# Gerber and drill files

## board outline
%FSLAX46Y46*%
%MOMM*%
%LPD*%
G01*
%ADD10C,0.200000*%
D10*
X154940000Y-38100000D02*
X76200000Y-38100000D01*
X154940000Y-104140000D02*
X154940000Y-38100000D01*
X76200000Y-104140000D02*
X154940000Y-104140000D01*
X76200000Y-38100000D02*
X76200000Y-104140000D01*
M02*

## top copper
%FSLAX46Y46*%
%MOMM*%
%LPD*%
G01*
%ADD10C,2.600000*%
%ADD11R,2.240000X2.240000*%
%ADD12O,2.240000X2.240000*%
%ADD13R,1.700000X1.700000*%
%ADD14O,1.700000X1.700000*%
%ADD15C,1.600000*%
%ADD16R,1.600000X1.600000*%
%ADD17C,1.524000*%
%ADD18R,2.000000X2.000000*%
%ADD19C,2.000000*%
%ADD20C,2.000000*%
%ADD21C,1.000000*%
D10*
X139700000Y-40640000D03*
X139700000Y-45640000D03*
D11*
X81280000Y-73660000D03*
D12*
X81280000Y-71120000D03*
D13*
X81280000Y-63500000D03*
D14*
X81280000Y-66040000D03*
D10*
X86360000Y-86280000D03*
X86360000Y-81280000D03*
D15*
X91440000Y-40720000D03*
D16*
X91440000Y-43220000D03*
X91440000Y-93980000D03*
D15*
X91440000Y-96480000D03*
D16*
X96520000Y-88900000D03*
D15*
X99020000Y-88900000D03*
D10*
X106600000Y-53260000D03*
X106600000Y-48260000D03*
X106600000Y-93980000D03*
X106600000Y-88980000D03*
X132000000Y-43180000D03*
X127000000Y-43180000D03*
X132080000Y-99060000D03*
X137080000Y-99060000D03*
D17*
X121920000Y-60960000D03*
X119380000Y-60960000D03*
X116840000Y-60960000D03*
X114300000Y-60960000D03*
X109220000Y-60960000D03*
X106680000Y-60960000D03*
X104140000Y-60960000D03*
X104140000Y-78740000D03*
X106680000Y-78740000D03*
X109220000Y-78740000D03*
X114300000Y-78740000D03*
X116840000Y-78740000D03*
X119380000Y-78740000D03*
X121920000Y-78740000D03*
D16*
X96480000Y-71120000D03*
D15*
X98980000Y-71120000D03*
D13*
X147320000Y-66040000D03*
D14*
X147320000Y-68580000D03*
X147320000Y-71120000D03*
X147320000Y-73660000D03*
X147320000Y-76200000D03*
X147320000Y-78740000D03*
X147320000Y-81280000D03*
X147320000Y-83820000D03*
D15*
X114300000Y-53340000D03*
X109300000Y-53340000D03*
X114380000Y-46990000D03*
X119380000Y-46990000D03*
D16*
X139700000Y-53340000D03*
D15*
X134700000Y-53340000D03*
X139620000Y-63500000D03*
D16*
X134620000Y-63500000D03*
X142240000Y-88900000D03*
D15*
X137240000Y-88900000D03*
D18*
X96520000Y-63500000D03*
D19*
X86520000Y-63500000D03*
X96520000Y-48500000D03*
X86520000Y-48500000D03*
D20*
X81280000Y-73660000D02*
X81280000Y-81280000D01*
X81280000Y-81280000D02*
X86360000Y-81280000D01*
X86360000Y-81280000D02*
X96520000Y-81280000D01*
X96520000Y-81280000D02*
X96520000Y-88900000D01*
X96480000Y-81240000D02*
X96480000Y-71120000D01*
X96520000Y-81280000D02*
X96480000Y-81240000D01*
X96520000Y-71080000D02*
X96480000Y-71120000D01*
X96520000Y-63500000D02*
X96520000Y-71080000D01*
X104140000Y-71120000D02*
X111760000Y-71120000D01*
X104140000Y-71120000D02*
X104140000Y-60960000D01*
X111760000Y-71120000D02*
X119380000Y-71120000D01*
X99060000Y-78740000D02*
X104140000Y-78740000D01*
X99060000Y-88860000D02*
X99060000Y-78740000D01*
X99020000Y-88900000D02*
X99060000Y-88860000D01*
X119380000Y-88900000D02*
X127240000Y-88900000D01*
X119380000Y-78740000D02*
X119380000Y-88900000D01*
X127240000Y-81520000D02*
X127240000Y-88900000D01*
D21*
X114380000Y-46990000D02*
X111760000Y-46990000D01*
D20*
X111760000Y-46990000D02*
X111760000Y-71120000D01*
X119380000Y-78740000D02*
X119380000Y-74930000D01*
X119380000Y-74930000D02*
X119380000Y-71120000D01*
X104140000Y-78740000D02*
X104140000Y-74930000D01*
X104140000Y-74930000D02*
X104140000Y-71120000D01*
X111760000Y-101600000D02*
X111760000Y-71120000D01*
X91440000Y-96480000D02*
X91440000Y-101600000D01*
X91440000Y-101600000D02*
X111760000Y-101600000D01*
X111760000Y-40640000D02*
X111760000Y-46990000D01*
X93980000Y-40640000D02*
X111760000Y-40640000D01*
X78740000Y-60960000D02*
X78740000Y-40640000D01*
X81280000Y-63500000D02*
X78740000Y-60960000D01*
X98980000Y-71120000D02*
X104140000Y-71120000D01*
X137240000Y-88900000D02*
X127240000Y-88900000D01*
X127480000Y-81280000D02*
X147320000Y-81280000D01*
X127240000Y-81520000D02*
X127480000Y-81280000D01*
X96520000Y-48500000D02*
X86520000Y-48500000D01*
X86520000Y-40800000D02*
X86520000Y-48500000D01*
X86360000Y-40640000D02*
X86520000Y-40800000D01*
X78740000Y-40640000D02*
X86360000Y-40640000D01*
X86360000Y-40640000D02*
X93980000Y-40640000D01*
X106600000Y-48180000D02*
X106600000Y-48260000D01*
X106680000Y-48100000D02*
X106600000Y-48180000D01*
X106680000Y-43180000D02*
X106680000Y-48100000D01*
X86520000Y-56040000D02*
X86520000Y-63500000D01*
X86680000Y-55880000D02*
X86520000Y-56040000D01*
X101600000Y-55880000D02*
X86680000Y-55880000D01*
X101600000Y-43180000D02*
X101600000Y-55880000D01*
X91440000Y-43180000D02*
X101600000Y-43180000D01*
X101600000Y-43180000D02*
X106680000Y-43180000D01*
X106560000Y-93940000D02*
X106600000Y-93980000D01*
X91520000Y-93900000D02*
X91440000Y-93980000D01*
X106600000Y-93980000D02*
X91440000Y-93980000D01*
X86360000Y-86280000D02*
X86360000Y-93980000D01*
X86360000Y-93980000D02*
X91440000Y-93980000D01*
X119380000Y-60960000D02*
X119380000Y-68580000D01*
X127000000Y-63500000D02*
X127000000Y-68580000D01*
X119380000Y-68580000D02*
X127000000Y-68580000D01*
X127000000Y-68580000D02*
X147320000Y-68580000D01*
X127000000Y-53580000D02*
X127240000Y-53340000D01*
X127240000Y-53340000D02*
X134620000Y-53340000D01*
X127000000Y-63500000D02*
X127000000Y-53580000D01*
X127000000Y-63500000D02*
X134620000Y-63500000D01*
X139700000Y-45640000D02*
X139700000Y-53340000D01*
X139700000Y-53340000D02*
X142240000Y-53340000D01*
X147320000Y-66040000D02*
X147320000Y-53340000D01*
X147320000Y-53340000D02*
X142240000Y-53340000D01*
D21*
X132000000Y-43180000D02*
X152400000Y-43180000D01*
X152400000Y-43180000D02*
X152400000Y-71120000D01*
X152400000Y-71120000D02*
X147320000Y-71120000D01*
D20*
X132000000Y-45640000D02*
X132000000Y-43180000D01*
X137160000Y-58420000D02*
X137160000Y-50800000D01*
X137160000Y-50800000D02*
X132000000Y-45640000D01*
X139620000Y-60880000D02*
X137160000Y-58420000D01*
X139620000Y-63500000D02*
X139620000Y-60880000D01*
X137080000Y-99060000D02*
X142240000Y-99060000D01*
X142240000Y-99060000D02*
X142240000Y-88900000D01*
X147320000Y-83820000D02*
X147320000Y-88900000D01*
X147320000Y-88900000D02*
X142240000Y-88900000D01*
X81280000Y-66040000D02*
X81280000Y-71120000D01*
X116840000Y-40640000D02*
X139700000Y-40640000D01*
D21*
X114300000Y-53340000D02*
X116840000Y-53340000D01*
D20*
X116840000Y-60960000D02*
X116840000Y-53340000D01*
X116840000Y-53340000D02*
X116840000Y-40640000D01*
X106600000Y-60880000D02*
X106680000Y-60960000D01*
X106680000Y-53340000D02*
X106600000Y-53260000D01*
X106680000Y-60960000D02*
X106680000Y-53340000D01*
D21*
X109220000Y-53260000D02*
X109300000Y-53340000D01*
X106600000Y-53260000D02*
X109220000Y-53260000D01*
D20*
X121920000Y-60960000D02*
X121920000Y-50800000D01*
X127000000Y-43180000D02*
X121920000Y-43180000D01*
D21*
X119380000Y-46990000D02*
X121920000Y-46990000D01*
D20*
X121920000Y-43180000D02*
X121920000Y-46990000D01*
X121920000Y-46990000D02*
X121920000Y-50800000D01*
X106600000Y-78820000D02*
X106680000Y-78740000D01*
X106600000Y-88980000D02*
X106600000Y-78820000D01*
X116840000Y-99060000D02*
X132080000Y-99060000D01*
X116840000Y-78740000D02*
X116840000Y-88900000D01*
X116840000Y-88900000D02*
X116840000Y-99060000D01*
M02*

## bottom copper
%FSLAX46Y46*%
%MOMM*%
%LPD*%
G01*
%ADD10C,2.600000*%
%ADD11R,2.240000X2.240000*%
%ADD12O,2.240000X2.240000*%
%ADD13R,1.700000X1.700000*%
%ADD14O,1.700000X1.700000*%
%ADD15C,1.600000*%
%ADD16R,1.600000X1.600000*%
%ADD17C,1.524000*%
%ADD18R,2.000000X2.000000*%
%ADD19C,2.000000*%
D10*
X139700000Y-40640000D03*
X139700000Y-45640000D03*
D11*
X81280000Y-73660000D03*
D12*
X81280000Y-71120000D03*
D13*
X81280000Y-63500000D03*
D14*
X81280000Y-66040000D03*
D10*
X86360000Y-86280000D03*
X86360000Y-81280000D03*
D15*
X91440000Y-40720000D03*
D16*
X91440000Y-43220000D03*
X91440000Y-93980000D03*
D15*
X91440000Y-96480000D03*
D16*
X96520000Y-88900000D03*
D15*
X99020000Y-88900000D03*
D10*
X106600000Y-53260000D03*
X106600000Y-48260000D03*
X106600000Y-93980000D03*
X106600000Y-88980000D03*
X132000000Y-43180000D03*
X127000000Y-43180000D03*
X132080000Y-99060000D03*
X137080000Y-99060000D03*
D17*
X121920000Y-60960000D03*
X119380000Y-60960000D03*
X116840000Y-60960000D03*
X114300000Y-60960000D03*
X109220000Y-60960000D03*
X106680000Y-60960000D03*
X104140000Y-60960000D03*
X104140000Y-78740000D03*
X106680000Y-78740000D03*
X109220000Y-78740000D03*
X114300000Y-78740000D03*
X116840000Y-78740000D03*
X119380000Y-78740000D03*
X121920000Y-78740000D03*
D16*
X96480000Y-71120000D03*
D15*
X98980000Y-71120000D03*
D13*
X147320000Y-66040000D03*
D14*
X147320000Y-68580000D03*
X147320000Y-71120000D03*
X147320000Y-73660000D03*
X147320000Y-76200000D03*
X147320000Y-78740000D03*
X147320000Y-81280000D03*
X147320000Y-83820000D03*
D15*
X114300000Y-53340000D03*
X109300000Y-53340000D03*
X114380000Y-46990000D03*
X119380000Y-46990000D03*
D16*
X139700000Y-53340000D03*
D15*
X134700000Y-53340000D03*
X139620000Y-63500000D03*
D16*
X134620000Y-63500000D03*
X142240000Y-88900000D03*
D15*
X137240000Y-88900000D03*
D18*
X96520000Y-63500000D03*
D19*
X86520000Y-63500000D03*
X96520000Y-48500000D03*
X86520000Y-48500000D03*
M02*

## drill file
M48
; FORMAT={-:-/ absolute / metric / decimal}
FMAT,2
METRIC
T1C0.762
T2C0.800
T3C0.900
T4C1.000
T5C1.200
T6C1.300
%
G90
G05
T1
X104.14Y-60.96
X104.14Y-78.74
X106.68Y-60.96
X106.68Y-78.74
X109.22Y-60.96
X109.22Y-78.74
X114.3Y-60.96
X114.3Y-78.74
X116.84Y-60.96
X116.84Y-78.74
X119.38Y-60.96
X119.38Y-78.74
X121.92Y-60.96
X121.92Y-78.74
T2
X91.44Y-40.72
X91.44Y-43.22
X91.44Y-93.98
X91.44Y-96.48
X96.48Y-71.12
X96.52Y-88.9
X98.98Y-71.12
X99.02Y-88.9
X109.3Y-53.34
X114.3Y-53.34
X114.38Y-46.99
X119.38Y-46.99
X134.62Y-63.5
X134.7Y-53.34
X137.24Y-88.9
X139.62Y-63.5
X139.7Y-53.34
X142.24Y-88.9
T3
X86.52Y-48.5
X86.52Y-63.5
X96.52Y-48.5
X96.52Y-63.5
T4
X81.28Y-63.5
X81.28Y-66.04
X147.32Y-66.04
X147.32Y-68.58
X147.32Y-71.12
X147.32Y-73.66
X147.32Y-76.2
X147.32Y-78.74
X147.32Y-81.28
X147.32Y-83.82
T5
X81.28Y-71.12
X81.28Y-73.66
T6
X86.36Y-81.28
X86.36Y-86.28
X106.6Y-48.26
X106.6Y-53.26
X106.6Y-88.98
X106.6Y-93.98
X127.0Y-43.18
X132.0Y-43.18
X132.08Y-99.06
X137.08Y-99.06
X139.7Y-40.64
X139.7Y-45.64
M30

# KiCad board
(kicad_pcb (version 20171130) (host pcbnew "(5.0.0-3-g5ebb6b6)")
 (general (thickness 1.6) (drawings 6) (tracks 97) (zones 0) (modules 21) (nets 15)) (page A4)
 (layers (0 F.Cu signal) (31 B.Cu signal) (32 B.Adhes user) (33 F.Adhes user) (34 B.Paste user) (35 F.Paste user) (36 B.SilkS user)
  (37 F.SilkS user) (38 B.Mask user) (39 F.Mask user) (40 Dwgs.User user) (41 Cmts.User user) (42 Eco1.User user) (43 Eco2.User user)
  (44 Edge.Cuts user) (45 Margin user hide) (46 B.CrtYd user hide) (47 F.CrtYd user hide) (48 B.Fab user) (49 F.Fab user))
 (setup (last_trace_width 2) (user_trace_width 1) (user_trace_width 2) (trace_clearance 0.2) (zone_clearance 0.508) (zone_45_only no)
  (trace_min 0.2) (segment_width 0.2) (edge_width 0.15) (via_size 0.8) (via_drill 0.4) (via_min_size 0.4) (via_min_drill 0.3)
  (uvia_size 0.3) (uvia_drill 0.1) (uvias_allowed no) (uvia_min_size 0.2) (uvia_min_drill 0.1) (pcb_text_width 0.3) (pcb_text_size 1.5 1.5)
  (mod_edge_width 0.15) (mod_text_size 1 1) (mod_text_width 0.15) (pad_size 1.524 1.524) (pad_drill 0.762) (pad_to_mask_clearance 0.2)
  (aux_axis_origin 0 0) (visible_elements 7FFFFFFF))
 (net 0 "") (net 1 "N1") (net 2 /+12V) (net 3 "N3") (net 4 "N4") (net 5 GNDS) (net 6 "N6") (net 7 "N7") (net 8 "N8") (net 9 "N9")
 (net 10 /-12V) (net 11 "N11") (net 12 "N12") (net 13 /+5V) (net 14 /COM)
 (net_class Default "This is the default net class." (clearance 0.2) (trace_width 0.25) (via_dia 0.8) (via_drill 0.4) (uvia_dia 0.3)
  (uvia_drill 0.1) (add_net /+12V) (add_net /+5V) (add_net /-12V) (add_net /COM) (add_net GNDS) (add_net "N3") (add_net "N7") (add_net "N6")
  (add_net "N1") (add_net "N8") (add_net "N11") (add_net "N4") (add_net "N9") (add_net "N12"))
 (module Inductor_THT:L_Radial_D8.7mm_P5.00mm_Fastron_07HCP (layer F.Cu) (at 139.7 40.64 270)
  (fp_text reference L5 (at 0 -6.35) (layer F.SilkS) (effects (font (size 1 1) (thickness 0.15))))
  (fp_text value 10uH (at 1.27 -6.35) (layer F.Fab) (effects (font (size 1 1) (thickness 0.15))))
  (pad 1 thru_hole circle (at 0 0 270) (size 2.6 2.6) (drill 1.3) (layers *.Cu *.Mask) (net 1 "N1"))
  (pad 2 thru_hole circle (at 5 0 270) (size 2.6 2.6) (drill 1.3) (layers *.Cu *.Mask) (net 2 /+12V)))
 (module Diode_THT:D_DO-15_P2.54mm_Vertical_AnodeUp (layer F.Cu) (at 81.28 73.66 90)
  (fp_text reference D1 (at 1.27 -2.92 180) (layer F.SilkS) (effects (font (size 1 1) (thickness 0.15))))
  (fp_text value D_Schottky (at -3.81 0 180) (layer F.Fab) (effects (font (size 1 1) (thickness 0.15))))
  (pad 1 thru_hole rect (at 0 0 90) (size 2.24 2.24) (drill 1.2) (layers *.Cu *.Mask) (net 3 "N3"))
  (pad 2 thru_hole oval (at 2.54 0 90) (size 2.24 2.24) (drill 1.2) (layers *.Cu *.Mask) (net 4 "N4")))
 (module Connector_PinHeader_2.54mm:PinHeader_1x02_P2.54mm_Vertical (layer F.Cu) (at 81.28 63.5)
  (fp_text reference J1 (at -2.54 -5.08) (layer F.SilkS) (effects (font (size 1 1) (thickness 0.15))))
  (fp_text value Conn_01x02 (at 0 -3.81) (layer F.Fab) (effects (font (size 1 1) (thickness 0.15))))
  (pad 1 thru_hole rect (at 0 0) (size 1.7 1.7) (drill 1) (layers *.Cu *.Mask) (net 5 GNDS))
  (pad 2 thru_hole oval (at 0 2.54) (size 1.7 1.7) (drill 1) (layers *.Cu *.Mask) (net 4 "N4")))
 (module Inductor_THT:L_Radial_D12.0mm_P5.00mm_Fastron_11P (layer F.Cu) (at 86.36 81.28 270)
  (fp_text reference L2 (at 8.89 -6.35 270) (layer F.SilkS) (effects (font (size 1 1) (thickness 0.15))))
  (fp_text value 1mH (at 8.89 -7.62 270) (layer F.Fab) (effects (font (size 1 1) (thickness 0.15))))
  (pad 2 thru_hole circle (at 5 0 270) (size 2.6 2.6) (drill 1.3) (layers *.Cu *.Mask) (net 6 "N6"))
  (pad 1 thru_hole circle (at 0 0 270) (size 2.6 2.6) (drill 1.3) (layers *.Cu *.Mask) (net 3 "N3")))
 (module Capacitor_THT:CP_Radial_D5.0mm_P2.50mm (layer F.Cu) (at 91.44 43.22 90)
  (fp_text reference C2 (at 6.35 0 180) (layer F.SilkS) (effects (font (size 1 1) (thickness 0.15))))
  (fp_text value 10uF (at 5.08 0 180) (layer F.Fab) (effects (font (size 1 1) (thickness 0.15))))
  (pad 2 thru_hole circle (at 2.5 0 90) (size 1.6 1.6) (drill 0.8) (layers *.Cu *.Mask) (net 5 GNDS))
  (pad 1 thru_hole rect (at 0 0 90) (size 1.6 1.6) (drill 0.8) (layers *.Cu *.Mask) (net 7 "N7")))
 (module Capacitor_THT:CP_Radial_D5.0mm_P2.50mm (layer F.Cu) (at 91.44 93.98 270)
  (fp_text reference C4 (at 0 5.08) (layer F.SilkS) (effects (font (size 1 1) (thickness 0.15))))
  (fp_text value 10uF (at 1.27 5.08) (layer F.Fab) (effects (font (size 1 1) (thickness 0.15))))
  (pad 1 thru_hole rect (at 0 0 270) (size 1.6 1.6) (drill 0.8) (layers *.Cu *.Mask) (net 6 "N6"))
  (pad 2 thru_hole circle (at 2.5 0 270) (size 1.6 1.6) (drill 0.8) (layers *.Cu *.Mask) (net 5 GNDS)))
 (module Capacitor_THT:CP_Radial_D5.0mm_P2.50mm (layer F.Cu) (at 96.52 88.9)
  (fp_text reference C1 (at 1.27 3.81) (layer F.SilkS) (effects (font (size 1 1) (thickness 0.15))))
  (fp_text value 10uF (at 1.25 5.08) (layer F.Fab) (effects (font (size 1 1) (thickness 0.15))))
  (pad 1 thru_hole rect (at 0 0) (size 1.6 1.6) (drill 0.8) (layers *.Cu *.Mask) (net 3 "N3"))
  (pad 2 thru_hole circle (at 2.5 0) (size 1.6 1.6) (drill 0.8) (layers *.Cu *.Mask) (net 5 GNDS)))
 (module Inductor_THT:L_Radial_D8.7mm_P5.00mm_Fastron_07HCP (layer F.Cu) (at 106.6 48.26 270)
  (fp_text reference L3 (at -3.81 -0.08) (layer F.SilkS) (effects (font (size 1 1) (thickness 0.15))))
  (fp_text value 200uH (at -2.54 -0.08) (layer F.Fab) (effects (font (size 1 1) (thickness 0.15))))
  (pad 2 thru_hole circle (at 5 0 270) (size 2.6 2.6) (drill 1.3) (layers *.Cu *.Mask) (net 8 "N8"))
  (pad 1 thru_hole circle (at 0 0 270) (size 2.6 2.6) (drill 1.3) (layers *.Cu *.Mask) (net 7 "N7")))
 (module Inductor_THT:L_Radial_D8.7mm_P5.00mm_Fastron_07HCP (layer F.Cu) (at 106.6 93.98 90)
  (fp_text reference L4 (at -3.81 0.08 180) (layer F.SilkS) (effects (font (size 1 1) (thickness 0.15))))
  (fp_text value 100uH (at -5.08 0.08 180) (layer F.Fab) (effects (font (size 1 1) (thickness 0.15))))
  (pad 1 thru_hole circle (at 0 0 90) (size 2.6 2.6) (drill 1.3) (layers *.Cu *.Mask) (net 6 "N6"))
  (pad 2 thru_hole circle (at 5 0 90) (size 2.6 2.6) (drill 1.3) (layers *.Cu *.Mask) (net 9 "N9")))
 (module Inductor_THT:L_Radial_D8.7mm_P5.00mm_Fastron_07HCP (layer F.Cu) (at 127 43.18)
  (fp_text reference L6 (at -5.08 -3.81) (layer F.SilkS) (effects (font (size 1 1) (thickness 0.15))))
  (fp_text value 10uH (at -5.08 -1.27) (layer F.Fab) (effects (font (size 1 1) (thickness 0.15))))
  (pad 2 thru_hole circle (at 5 0) (size 2.6 2.6) (drill 1.3) (layers *.Cu *.Mask) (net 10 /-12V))
  (pad 1 thru_hole circle (at 0 0) (size 2.6 2.6) (drill 1.3) (layers *.Cu *.Mask) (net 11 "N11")))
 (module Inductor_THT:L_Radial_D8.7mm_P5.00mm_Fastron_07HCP (layer F.Cu) (at 132.08 99.06)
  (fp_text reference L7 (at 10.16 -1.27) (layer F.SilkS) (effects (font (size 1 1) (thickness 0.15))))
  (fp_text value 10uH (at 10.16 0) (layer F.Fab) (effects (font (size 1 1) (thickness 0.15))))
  (pad 1 thru_hole circle (at 0 0) (size 2.6 2.6) (drill 1.3) (layers *.Cu *.Mask) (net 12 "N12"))
  (pad 2 thru_hole circle (at 5 0) (size 2.6 2.6) (drill 1.3) (layers *.Cu *.Mask) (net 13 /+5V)))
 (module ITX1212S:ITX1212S (layer F.Cu) (at 111.76 60.96)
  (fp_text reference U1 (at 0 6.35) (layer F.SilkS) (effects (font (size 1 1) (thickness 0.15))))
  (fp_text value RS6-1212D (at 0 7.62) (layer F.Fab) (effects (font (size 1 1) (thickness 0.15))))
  (pad 8 thru_hole circle (at 10.16 0) (size 1.524 1.524) (drill 0.762) (layers *.Cu *.Mask) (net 11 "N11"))
  (pad 7 thru_hole circle (at 7.62 0) (size 1.524 1.524) (drill 0.762) (layers *.Cu *.Mask) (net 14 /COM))
  (pad 6 thru_hole circle (at 5.08 0) (size 1.524 1.524) (drill 0.762) (layers *.Cu *.Mask) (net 1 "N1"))
  (pad 5 thru_hole circle (at 2.54 0) (size 1.524 1.524) (drill 0.762) (layers *.Cu *.Mask))
  (pad 3 thru_hole circle (at -2.54 0) (size 1.524 1.524) (drill 0.762) (layers *.Cu *.Mask))
  (pad 2 thru_hole circle (at -5.08 0) (size 1.524 1.524) (drill 0.762) (layers *.Cu *.Mask) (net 8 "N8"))
  (pad 1 thru_hole circle (at -7.62 0) (size 1.524 1.524) (drill 0.762) (layers *.Cu *.Mask) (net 5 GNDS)))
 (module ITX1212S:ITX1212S (layer F.Cu) (at 111.76 78.74)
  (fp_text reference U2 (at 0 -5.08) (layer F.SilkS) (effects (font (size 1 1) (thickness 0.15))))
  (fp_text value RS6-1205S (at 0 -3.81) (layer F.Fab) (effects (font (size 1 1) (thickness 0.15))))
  (pad 1 thru_hole circle (at -7.62 0) (size 1.524 1.524) (drill 0.762) (layers *.Cu *.Mask) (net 5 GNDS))
  (pad 2 thru_hole circle (at -5.08 0) (size 1.524 1.524) (drill 0.762) (layers *.Cu *.Mask) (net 9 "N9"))
  (pad 3 thru_hole circle (at -2.54 0) (size 1.524 1.524) (drill 0.762) (layers *.Cu *.Mask))
  (pad 5 thru_hole circle (at 2.54 0) (size 1.524 1.524) (drill 0.762) (layers *.Cu *.Mask))
  (pad 6 thru_hole circle (at 5.08 0) (size 1.524 1.524) (drill 0.762) (layers *.Cu *.Mask) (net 12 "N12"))
  (pad 7 thru_hole circle (at 7.62 0) (size 1.524 1.524) (drill 0.762) (layers *.Cu *.Mask) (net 5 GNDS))
  (pad 8 thru_hole circle (at 10.16 0) (size 1.524 1.524) (drill 0.762) (layers *.Cu *.Mask)))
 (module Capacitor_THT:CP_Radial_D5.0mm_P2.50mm (layer F.Cu) (at 96.48 71.12)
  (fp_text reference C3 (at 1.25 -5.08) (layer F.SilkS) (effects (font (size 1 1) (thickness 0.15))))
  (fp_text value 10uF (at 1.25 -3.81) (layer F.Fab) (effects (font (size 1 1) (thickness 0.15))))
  (pad 1 thru_hole rect (at 0 0) (size 1.6 1.6) (drill 0.8) (layers *.Cu *.Mask) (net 3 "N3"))
  (pad 2 thru_hole circle (at 2.5 0) (size 1.6 1.6) (drill 0.8) (layers *.Cu *.Mask) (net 5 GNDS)))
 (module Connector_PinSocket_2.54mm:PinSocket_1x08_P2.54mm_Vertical (layer F.Cu) (at 147.32 66.04)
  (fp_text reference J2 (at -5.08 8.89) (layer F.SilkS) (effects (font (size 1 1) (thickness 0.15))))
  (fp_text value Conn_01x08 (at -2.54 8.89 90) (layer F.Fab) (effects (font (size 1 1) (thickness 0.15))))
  (pad 1 thru_hole rect (at 0 0) (size 1.7 1.7) (drill 1) (layers *.Cu *.Mask) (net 2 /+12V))
  (pad 2 thru_hole oval (at 0 2.54) (size 1.7 1.7) (drill 1) (layers *.Cu *.Mask) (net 14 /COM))
  (pad 3 thru_hole oval (at 0 5.08) (size 1.7 1.7) (drill 1) (layers *.Cu *.Mask) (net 10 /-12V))
  (pad 4 thru_hole oval (at 0 7.62) (size 1.7 1.7) (drill 1) (layers *.Cu *.Mask))
  (pad 5 thru_hole oval (at 0 10.16) (size 1.7 1.7) (drill 1) (layers *.Cu *.Mask))
  (pad 6 thru_hole oval (at 0 12.7) (size 1.7 1.7) (drill 1) (layers *.Cu *.Mask))
  (pad 7 thru_hole oval (at 0 15.24) (size 1.7 1.7) (drill 1) (layers *.Cu *.Mask) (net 5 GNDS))
  (pad 8 thru_hole oval (at 0 17.78) (size 1.7 1.7) (drill 1) (layers *.Cu *.Mask) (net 13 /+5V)))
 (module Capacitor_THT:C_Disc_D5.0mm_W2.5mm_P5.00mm (layer B.Cu) (at 114.3 53.34 180)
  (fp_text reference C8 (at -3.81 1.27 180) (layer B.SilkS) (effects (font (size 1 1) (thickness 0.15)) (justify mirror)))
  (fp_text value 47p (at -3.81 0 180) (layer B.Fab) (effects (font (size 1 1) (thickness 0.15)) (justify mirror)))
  (pad 1 thru_hole circle (at 0 0 180) (size 1.6 1.6) (drill 0.8) (layers *.Cu *.Mask) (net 1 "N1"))
  (pad 2 thru_hole circle (at 5 0 180) (size 1.6 1.6) (drill 0.8) (layers *.Cu *.Mask) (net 8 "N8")))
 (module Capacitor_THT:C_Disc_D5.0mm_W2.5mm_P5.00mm (layer B.Cu) (at 119.38 46.99 180)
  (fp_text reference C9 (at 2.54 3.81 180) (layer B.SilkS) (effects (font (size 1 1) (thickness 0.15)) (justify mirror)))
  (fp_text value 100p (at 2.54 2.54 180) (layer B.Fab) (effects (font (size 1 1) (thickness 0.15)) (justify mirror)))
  (pad 2 thru_hole circle (at 5 0 180) (size 1.6 1.6) (drill 0.8) (layers *.Cu *.Mask) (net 5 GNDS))
  (pad 1 thru_hole circle (at 0 0 180) (size 1.6 1.6) (drill 0.8) (layers *.Cu *.Mask) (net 11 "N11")))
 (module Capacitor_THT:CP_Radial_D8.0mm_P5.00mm (layer F.Cu) (at 139.7 53.34 180)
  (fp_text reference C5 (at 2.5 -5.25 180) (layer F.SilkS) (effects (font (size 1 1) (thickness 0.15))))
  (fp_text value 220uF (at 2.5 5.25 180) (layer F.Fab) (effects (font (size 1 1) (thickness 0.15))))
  (pad 1 thru_hole rect (at 0 0 180) (size 1.6 1.6) (drill 0.8) (layers *.Cu *.Mask) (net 2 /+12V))
  (pad 2 thru_hole circle (at 5 0 180) (size 1.6 1.6) (drill 0.8) (layers *.Cu *.Mask) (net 14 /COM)))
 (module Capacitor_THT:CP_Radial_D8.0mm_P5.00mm (layer F.Cu) (at 134.62 63.5)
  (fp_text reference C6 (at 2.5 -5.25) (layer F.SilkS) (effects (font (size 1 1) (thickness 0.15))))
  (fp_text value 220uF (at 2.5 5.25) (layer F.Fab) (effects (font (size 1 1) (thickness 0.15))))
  (pad 2 thru_hole circle (at 5 0) (size 1.6 1.6) (drill 0.8) (layers *.Cu *.Mask) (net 10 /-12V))
  (pad 1 thru_hole rect (at 0 0) (size 1.6 1.6) (drill 0.8) (layers *.Cu *.Mask) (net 14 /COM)))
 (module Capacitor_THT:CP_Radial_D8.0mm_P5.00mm (layer F.Cu) (at 142.24 88.9 180)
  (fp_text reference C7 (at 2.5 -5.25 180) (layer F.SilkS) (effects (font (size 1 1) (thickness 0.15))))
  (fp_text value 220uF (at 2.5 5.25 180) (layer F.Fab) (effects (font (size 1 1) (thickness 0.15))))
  (pad 1 thru_hole rect (at 0 0 180) (size 1.6 1.6) (drill 0.8) (layers *.Cu *.Mask) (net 13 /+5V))
  (pad 2 thru_hole circle (at 5 0 180) (size 1.6 1.6) (drill 0.8) (layers *.Cu *.Mask) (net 5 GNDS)))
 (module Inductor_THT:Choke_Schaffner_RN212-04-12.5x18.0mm (layer F.Cu) (at 96.52 63.5 180)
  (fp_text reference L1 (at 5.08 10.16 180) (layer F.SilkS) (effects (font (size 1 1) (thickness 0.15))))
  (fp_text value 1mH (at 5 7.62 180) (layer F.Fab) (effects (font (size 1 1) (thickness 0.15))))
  (pad 1 thru_hole rect (at 0 0 180) (size 2 2) (drill 0.9) (layers *.Cu *.Mask) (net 3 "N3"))
  (pad 2 thru_hole circle (at 10 0 180) (size 2 2) (drill 0.9) (layers *.Cu *.Mask) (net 7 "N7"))
  (pad 3 thru_hole circle (at 0 15 180) (size 2 2) (drill 0.9) (layers *.Cu *.Mask) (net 5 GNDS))
  (pad 4 thru_hole circle (at 10 15 180) (size 2 2) (drill 0.9) (layers *.Cu *.Mask) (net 5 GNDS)))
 (gr_line (start 154.94 38.1) (end 76.2 38.1) (layer Edge.Cuts) (width 0.2))
 (gr_line (start 154.94 104.14) (end 154.94 38.1) (layer Edge.Cuts) (width 0.2))
 (gr_line (start 76.2 104.14) (end 154.94 104.14) (layer Edge.Cuts) (width 0.2))
 (gr_line (start 76.2 38.1) (end 76.2 104.14) (layer Edge.Cuts) (width 0.2))
 (segment (start 81.28 73.66) (end 81.28 81.28) (width 2) (layer F.Cu) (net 3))
 (segment (start 81.28 81.28) (end 86.36 81.28) (width 2) (layer F.Cu) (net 3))
 (segment (start 86.36 81.28) (end 96.52 81.28) (width 2) (layer F.Cu) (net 3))
 (segment (start 96.52 81.28) (end 96.52 88.9) (width 2) (layer F.Cu) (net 3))
 (segment (start 96.48 81.24) (end 96.48 71.12) (width 2) (layer F.Cu) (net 3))
 (segment (start 96.52 81.28) (end 96.48 81.24) (width 2) (layer F.Cu) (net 3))
 (segment (start 96.52 71.08) (end 96.48 71.12) (width 2) (layer F.Cu) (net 3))
 (segment (start 96.52 63.5) (end 96.52 71.08) (width 2) (layer F.Cu) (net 3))
 (segment (start 104.14 71.12) (end 111.76 71.12) (width 2) (layer F.Cu) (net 5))
 (segment (start 104.14 71.12) (end 104.14 60.96) (width 2) (layer F.Cu) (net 5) (status 20))
 (segment (start 111.76 71.12) (end 119.38 71.12) (width 2) (layer F.Cu) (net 5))
 (segment (start 99.06 78.74) (end 104.14 78.74) (width 2) (layer F.Cu) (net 5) (status 20))
 (segment (start 99.06 88.86) (end 99.06 78.74) (width 2) (layer F.Cu) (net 5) (status 10))
 (segment (start 99.02 88.9) (end 99.06 88.86) (width 2) (layer F.Cu) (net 5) (status 30))
 (segment (start 119.38 88.9) (end 127.24 88.9) (width 2) (layer F.Cu) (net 5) (status 20))
 (segment (start 119.38 78.74) (end 119.38 88.9) (width 2) (layer F.Cu) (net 5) (status 10))
 (segment (start 127.24 81.52) (end 127.24 88.9) (width 2) (layer F.Cu) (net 5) (status 20))
 (segment (start 114.38 46.99) (end 111.76 46.99) (width 1) (layer F.Cu) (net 5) (status 10))
 (segment (start 111.76 46.99) (end 111.76 71.12) (width 2) (layer F.Cu) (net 5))
 (segment (start 119.38 78.74) (end 119.38 74.93) (width 2) (layer F.Cu) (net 5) (status 10))
 (segment (start 119.38 74.93) (end 119.38 71.12) (width 2) (layer F.Cu) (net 5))
 (segment (start 104.14 78.74) (end 104.14 74.93) (width 2) (layer F.Cu) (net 5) (status 10))
 (segment (start 104.14 74.93) (end 104.14 71.12) (width 2) (layer F.Cu) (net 5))
 (segment (start 111.76 101.6) (end 111.76 71.12) (width 2) (layer F.Cu) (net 5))
 (segment (start 91.44 96.48) (end 91.44 101.6) (width 2) (layer F.Cu) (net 5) (status 10))
 (segment (start 91.44 101.6) (end 111.76 101.6) (width 2) (layer F.Cu) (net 5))
 (segment (start 111.76 40.64) (end 111.76 46.99) (width 2) (layer F.Cu) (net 5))
 (segment (start 93.98 40.64) (end 111.76 40.64) (width 2) (layer F.Cu) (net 5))
 (segment (start 78.74 60.96) (end 78.74 40.64) (width 2) (layer F.Cu) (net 5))
 (segment (start 81.28 63.5) (end 78.74 60.96) (width 2) (layer F.Cu) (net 5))
 (segment (start 98.98 71.12) (end 104.14 71.12) (width 2) (layer F.Cu) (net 5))
 (segment (start 137.24 88.9) (end 127.24 88.9) (width 2) (layer F.Cu) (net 5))
 (segment (start 127.48 81.28) (end 147.32 81.28) (width 2) (layer F.Cu) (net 5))
 (segment (start 127.24 81.52) (end 127.48 81.28) (width 2) (layer F.Cu) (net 5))
 (segment (start 96.52 48.5) (end 86.52 48.5) (width 2) (layer F.Cu) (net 5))
 (segment (start 86.52 40.8) (end 86.52 48.5) (width 2) (layer F.Cu) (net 5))
 (segment (start 86.36 40.64) (end 86.52 40.8) (width 2) (layer F.Cu) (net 5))
 (segment (start 78.74 40.64) (end 86.36 40.64) (width 2) (layer F.Cu) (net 5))
 (segment (start 86.36 40.64) (end 93.98 40.64) (width 2) (layer F.Cu) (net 5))
 (segment (start 106.6 48.18) (end 106.6 48.26) (width 2) (layer F.Cu) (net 7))
 (segment (start 106.68 48.1) (end 106.6 48.18) (width 2) (layer F.Cu) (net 7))
 (segment (start 106.68 43.18) (end 106.68 48.1) (width 2) (layer F.Cu) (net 7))
 (segment (start 86.52 56.04) (end 86.52 63.5) (width 2) (layer F.Cu) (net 7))
 (segment (start 86.68 55.88) (end 86.52 56.04) (width 2) (layer F.Cu) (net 7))
 (segment (start 101.6 55.88) (end 86.68 55.88) (width 2) (layer F.Cu) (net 7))
 (segment (start 101.6 43.18) (end 101.6 55.88) (width 2) (layer F.Cu) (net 7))
 (segment (start 91.44 43.18) (end 101.6 43.18) (width 2) (layer F.Cu) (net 7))
 (segment (start 101.6 43.18) (end 106.68 43.18) (width 2) (layer F.Cu) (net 7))
 (segment (start 106.56 93.94) (end 106.6 93.98) (width 2) (layer F.Cu) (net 6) (status 30))
 (segment (start 91.52 93.9) (end 91.44 93.98) (width 2) (layer F.Cu) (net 6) (status 30))
 (segment (start 106.6 93.98) (end 91.44 93.98) (width 2) (layer F.Cu) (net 6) (status 30))
 (segment (start 86.36 86.28) (end 86.36 93.98) (width 2) (layer F.Cu) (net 6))
 (segment (start 86.36 93.98) (end 91.44 93.98) (width 2) (layer F.Cu) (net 6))
 (segment (start 119.38 60.96) (end 119.38 68.58) (width 2) (layer F.Cu) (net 14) (status 10))
 (segment (start 127 63.5) (end 127 68.58) (width 2) (layer F.Cu) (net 14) (status 10))
 (segment (start 119.38 68.58) (end 127 68.58) (width 2) (layer F.Cu) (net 14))
 (segment (start 127 68.58) (end 147.32 68.58) (width 2) (layer F.Cu) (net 14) (status 20))
 (segment (start 127 53.58) (end 127.24 53.34) (width 2) (layer F.Cu) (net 14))
 (segment (start 127.24 53.34) (end 134.62 53.34) (width 2) (layer F.Cu) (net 14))
 (segment (start 127 63.5) (end 127 53.58) (width 2) (layer F.Cu) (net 14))
 (segment (start 127 63.5) (end 134.62 63.5) (width 2) (layer F.Cu) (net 14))
 (segment (start 139.7 45.64) (end 139.7 53.34) (width 2) (layer F.Cu) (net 2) (status 10))
 (segment (start 139.7 53.34) (end 142.24 53.34) (width 2) (layer F.Cu) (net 2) (status 20))
 (segment (start 147.32 66.04) (end 147.32 53.34) (width 2) (layer F.Cu) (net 2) (status 10))
 (segment (start 147.32 53.34) (end 142.24 53.34) (width 2) (layer F.Cu) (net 2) (status 20))
 (segment (start 132 43.18) (end 152.4 43.18) (width 1) (layer F.Cu) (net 10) (status 10))
 (segment (start 152.4 43.18) (end 152.4 71.12) (width 1) (layer F.Cu) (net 10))
 (segment (start 152.4 71.12) (end 147.32 71.12) (width 1) (layer F.Cu) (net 10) (status 20))
 (segment (start 132 45.64) (end 132 43.18) (width 2) (layer F.Cu) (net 10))
 (segment (start 137.16 58.42) (end 137.16 50.8) (width 2) (layer F.Cu) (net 10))
 (segment (start 137.16 50.8) (end 132 45.64) (width 2) (layer F.Cu) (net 10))
 (segment (start 139.62 60.88) (end 137.16 58.42) (width 2) (layer F.Cu) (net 10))
 (segment (start 139.62 63.5) (end 139.62 60.88) (width 2) (layer F.Cu) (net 10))
 (segment (start 137.08 99.06) (end 142.24 99.06) (width 2) (layer F.Cu) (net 13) (status 10))
 (segment (start 142.24 99.06) (end 142.24 88.9) (width 2) (layer F.Cu) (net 13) (status 20))
 (segment (start 147.32 83.82) (end 147.32 88.9) (width 2) (layer F.Cu) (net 13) (status 10))
 (segment (start 147.32 88.9) (end 142.24 88.9) (width 2) (layer F.Cu) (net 13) (status 20))
 (segment (start 81.28 66.04) (end 81.28 71.12) (width 2) (layer F.Cu) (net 4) (status 30))
 (segment (start 116.84 40.64) (end 139.7 40.64) (width 2) (layer F.Cu) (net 1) (status 20))
 (segment (start 114.3 53.34) (end 116.84 53.34) (width 1) (layer F.Cu) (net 1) (status 10))
 (segment (start 116.84 60.96) (end 116.84 53.34) (width 2) (layer F.Cu) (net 1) (status 10))
 (segment (start 116.84 53.34) (end 116.84 40.64) (width 2) (layer F.Cu) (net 1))
 (segment (start 106.6 60.88) (end 106.68 60.96) (width 2) (layer F.Cu) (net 8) (status 30))
 (segment (start 106.68 53.34) (end 106.6 53.26) (width 2) (layer F.Cu) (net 8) (status 30))
 (segment (start 106.68 60.96) (end 106.68 53.34) (width 2) (layer F.Cu) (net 8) (status 30))
 (segment (start 109.22 53.26) (end 109.3 53.34) (width 1) (layer F.Cu) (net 8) (status 30))
 (segment (start 106.6 53.26) (end 109.22 53.26) (width 1) (layer F.Cu) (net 8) (status 30))
 (segment (start 121.92 60.96) (end 121.92 50.8) (width 2) (layer F.Cu) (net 11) (status 10))
 (segment (start 127 43.18) (end 121.92 43.18) (width 2) (layer F.Cu) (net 11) (status 10))
 (segment (start 119.38 46.99) (end 121.92 46.99) (width 1) (layer F.Cu) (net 11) (status 10))
 (segment (start 121.92 43.18) (end 121.92 46.99) (width 2) (layer F.Cu) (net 11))
 (segment (start 121.92 46.99) (end 121.92 50.8) (width 2) (layer F.Cu) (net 11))
 (segment (start 106.6 78.82) (end 106.68 78.74) (width 2) (layer F.Cu) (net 9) (status 30))
 (segment (start 106.6 88.98) (end 106.6 78.82) (width 2) (layer F.Cu) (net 9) (status 30))
 (segment (start 116.84 99.06) (end 132.08 99.06) (width 2) (layer F.Cu) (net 12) (status 20))
 (segment (start 116.84 78.74) (end 116.84 88.9) (width 2) (layer F.Cu) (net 12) (status 10))
 (segment (start 116.84 88.9) (end 116.84 99.06) (width 2) (layer F.Cu) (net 12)))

